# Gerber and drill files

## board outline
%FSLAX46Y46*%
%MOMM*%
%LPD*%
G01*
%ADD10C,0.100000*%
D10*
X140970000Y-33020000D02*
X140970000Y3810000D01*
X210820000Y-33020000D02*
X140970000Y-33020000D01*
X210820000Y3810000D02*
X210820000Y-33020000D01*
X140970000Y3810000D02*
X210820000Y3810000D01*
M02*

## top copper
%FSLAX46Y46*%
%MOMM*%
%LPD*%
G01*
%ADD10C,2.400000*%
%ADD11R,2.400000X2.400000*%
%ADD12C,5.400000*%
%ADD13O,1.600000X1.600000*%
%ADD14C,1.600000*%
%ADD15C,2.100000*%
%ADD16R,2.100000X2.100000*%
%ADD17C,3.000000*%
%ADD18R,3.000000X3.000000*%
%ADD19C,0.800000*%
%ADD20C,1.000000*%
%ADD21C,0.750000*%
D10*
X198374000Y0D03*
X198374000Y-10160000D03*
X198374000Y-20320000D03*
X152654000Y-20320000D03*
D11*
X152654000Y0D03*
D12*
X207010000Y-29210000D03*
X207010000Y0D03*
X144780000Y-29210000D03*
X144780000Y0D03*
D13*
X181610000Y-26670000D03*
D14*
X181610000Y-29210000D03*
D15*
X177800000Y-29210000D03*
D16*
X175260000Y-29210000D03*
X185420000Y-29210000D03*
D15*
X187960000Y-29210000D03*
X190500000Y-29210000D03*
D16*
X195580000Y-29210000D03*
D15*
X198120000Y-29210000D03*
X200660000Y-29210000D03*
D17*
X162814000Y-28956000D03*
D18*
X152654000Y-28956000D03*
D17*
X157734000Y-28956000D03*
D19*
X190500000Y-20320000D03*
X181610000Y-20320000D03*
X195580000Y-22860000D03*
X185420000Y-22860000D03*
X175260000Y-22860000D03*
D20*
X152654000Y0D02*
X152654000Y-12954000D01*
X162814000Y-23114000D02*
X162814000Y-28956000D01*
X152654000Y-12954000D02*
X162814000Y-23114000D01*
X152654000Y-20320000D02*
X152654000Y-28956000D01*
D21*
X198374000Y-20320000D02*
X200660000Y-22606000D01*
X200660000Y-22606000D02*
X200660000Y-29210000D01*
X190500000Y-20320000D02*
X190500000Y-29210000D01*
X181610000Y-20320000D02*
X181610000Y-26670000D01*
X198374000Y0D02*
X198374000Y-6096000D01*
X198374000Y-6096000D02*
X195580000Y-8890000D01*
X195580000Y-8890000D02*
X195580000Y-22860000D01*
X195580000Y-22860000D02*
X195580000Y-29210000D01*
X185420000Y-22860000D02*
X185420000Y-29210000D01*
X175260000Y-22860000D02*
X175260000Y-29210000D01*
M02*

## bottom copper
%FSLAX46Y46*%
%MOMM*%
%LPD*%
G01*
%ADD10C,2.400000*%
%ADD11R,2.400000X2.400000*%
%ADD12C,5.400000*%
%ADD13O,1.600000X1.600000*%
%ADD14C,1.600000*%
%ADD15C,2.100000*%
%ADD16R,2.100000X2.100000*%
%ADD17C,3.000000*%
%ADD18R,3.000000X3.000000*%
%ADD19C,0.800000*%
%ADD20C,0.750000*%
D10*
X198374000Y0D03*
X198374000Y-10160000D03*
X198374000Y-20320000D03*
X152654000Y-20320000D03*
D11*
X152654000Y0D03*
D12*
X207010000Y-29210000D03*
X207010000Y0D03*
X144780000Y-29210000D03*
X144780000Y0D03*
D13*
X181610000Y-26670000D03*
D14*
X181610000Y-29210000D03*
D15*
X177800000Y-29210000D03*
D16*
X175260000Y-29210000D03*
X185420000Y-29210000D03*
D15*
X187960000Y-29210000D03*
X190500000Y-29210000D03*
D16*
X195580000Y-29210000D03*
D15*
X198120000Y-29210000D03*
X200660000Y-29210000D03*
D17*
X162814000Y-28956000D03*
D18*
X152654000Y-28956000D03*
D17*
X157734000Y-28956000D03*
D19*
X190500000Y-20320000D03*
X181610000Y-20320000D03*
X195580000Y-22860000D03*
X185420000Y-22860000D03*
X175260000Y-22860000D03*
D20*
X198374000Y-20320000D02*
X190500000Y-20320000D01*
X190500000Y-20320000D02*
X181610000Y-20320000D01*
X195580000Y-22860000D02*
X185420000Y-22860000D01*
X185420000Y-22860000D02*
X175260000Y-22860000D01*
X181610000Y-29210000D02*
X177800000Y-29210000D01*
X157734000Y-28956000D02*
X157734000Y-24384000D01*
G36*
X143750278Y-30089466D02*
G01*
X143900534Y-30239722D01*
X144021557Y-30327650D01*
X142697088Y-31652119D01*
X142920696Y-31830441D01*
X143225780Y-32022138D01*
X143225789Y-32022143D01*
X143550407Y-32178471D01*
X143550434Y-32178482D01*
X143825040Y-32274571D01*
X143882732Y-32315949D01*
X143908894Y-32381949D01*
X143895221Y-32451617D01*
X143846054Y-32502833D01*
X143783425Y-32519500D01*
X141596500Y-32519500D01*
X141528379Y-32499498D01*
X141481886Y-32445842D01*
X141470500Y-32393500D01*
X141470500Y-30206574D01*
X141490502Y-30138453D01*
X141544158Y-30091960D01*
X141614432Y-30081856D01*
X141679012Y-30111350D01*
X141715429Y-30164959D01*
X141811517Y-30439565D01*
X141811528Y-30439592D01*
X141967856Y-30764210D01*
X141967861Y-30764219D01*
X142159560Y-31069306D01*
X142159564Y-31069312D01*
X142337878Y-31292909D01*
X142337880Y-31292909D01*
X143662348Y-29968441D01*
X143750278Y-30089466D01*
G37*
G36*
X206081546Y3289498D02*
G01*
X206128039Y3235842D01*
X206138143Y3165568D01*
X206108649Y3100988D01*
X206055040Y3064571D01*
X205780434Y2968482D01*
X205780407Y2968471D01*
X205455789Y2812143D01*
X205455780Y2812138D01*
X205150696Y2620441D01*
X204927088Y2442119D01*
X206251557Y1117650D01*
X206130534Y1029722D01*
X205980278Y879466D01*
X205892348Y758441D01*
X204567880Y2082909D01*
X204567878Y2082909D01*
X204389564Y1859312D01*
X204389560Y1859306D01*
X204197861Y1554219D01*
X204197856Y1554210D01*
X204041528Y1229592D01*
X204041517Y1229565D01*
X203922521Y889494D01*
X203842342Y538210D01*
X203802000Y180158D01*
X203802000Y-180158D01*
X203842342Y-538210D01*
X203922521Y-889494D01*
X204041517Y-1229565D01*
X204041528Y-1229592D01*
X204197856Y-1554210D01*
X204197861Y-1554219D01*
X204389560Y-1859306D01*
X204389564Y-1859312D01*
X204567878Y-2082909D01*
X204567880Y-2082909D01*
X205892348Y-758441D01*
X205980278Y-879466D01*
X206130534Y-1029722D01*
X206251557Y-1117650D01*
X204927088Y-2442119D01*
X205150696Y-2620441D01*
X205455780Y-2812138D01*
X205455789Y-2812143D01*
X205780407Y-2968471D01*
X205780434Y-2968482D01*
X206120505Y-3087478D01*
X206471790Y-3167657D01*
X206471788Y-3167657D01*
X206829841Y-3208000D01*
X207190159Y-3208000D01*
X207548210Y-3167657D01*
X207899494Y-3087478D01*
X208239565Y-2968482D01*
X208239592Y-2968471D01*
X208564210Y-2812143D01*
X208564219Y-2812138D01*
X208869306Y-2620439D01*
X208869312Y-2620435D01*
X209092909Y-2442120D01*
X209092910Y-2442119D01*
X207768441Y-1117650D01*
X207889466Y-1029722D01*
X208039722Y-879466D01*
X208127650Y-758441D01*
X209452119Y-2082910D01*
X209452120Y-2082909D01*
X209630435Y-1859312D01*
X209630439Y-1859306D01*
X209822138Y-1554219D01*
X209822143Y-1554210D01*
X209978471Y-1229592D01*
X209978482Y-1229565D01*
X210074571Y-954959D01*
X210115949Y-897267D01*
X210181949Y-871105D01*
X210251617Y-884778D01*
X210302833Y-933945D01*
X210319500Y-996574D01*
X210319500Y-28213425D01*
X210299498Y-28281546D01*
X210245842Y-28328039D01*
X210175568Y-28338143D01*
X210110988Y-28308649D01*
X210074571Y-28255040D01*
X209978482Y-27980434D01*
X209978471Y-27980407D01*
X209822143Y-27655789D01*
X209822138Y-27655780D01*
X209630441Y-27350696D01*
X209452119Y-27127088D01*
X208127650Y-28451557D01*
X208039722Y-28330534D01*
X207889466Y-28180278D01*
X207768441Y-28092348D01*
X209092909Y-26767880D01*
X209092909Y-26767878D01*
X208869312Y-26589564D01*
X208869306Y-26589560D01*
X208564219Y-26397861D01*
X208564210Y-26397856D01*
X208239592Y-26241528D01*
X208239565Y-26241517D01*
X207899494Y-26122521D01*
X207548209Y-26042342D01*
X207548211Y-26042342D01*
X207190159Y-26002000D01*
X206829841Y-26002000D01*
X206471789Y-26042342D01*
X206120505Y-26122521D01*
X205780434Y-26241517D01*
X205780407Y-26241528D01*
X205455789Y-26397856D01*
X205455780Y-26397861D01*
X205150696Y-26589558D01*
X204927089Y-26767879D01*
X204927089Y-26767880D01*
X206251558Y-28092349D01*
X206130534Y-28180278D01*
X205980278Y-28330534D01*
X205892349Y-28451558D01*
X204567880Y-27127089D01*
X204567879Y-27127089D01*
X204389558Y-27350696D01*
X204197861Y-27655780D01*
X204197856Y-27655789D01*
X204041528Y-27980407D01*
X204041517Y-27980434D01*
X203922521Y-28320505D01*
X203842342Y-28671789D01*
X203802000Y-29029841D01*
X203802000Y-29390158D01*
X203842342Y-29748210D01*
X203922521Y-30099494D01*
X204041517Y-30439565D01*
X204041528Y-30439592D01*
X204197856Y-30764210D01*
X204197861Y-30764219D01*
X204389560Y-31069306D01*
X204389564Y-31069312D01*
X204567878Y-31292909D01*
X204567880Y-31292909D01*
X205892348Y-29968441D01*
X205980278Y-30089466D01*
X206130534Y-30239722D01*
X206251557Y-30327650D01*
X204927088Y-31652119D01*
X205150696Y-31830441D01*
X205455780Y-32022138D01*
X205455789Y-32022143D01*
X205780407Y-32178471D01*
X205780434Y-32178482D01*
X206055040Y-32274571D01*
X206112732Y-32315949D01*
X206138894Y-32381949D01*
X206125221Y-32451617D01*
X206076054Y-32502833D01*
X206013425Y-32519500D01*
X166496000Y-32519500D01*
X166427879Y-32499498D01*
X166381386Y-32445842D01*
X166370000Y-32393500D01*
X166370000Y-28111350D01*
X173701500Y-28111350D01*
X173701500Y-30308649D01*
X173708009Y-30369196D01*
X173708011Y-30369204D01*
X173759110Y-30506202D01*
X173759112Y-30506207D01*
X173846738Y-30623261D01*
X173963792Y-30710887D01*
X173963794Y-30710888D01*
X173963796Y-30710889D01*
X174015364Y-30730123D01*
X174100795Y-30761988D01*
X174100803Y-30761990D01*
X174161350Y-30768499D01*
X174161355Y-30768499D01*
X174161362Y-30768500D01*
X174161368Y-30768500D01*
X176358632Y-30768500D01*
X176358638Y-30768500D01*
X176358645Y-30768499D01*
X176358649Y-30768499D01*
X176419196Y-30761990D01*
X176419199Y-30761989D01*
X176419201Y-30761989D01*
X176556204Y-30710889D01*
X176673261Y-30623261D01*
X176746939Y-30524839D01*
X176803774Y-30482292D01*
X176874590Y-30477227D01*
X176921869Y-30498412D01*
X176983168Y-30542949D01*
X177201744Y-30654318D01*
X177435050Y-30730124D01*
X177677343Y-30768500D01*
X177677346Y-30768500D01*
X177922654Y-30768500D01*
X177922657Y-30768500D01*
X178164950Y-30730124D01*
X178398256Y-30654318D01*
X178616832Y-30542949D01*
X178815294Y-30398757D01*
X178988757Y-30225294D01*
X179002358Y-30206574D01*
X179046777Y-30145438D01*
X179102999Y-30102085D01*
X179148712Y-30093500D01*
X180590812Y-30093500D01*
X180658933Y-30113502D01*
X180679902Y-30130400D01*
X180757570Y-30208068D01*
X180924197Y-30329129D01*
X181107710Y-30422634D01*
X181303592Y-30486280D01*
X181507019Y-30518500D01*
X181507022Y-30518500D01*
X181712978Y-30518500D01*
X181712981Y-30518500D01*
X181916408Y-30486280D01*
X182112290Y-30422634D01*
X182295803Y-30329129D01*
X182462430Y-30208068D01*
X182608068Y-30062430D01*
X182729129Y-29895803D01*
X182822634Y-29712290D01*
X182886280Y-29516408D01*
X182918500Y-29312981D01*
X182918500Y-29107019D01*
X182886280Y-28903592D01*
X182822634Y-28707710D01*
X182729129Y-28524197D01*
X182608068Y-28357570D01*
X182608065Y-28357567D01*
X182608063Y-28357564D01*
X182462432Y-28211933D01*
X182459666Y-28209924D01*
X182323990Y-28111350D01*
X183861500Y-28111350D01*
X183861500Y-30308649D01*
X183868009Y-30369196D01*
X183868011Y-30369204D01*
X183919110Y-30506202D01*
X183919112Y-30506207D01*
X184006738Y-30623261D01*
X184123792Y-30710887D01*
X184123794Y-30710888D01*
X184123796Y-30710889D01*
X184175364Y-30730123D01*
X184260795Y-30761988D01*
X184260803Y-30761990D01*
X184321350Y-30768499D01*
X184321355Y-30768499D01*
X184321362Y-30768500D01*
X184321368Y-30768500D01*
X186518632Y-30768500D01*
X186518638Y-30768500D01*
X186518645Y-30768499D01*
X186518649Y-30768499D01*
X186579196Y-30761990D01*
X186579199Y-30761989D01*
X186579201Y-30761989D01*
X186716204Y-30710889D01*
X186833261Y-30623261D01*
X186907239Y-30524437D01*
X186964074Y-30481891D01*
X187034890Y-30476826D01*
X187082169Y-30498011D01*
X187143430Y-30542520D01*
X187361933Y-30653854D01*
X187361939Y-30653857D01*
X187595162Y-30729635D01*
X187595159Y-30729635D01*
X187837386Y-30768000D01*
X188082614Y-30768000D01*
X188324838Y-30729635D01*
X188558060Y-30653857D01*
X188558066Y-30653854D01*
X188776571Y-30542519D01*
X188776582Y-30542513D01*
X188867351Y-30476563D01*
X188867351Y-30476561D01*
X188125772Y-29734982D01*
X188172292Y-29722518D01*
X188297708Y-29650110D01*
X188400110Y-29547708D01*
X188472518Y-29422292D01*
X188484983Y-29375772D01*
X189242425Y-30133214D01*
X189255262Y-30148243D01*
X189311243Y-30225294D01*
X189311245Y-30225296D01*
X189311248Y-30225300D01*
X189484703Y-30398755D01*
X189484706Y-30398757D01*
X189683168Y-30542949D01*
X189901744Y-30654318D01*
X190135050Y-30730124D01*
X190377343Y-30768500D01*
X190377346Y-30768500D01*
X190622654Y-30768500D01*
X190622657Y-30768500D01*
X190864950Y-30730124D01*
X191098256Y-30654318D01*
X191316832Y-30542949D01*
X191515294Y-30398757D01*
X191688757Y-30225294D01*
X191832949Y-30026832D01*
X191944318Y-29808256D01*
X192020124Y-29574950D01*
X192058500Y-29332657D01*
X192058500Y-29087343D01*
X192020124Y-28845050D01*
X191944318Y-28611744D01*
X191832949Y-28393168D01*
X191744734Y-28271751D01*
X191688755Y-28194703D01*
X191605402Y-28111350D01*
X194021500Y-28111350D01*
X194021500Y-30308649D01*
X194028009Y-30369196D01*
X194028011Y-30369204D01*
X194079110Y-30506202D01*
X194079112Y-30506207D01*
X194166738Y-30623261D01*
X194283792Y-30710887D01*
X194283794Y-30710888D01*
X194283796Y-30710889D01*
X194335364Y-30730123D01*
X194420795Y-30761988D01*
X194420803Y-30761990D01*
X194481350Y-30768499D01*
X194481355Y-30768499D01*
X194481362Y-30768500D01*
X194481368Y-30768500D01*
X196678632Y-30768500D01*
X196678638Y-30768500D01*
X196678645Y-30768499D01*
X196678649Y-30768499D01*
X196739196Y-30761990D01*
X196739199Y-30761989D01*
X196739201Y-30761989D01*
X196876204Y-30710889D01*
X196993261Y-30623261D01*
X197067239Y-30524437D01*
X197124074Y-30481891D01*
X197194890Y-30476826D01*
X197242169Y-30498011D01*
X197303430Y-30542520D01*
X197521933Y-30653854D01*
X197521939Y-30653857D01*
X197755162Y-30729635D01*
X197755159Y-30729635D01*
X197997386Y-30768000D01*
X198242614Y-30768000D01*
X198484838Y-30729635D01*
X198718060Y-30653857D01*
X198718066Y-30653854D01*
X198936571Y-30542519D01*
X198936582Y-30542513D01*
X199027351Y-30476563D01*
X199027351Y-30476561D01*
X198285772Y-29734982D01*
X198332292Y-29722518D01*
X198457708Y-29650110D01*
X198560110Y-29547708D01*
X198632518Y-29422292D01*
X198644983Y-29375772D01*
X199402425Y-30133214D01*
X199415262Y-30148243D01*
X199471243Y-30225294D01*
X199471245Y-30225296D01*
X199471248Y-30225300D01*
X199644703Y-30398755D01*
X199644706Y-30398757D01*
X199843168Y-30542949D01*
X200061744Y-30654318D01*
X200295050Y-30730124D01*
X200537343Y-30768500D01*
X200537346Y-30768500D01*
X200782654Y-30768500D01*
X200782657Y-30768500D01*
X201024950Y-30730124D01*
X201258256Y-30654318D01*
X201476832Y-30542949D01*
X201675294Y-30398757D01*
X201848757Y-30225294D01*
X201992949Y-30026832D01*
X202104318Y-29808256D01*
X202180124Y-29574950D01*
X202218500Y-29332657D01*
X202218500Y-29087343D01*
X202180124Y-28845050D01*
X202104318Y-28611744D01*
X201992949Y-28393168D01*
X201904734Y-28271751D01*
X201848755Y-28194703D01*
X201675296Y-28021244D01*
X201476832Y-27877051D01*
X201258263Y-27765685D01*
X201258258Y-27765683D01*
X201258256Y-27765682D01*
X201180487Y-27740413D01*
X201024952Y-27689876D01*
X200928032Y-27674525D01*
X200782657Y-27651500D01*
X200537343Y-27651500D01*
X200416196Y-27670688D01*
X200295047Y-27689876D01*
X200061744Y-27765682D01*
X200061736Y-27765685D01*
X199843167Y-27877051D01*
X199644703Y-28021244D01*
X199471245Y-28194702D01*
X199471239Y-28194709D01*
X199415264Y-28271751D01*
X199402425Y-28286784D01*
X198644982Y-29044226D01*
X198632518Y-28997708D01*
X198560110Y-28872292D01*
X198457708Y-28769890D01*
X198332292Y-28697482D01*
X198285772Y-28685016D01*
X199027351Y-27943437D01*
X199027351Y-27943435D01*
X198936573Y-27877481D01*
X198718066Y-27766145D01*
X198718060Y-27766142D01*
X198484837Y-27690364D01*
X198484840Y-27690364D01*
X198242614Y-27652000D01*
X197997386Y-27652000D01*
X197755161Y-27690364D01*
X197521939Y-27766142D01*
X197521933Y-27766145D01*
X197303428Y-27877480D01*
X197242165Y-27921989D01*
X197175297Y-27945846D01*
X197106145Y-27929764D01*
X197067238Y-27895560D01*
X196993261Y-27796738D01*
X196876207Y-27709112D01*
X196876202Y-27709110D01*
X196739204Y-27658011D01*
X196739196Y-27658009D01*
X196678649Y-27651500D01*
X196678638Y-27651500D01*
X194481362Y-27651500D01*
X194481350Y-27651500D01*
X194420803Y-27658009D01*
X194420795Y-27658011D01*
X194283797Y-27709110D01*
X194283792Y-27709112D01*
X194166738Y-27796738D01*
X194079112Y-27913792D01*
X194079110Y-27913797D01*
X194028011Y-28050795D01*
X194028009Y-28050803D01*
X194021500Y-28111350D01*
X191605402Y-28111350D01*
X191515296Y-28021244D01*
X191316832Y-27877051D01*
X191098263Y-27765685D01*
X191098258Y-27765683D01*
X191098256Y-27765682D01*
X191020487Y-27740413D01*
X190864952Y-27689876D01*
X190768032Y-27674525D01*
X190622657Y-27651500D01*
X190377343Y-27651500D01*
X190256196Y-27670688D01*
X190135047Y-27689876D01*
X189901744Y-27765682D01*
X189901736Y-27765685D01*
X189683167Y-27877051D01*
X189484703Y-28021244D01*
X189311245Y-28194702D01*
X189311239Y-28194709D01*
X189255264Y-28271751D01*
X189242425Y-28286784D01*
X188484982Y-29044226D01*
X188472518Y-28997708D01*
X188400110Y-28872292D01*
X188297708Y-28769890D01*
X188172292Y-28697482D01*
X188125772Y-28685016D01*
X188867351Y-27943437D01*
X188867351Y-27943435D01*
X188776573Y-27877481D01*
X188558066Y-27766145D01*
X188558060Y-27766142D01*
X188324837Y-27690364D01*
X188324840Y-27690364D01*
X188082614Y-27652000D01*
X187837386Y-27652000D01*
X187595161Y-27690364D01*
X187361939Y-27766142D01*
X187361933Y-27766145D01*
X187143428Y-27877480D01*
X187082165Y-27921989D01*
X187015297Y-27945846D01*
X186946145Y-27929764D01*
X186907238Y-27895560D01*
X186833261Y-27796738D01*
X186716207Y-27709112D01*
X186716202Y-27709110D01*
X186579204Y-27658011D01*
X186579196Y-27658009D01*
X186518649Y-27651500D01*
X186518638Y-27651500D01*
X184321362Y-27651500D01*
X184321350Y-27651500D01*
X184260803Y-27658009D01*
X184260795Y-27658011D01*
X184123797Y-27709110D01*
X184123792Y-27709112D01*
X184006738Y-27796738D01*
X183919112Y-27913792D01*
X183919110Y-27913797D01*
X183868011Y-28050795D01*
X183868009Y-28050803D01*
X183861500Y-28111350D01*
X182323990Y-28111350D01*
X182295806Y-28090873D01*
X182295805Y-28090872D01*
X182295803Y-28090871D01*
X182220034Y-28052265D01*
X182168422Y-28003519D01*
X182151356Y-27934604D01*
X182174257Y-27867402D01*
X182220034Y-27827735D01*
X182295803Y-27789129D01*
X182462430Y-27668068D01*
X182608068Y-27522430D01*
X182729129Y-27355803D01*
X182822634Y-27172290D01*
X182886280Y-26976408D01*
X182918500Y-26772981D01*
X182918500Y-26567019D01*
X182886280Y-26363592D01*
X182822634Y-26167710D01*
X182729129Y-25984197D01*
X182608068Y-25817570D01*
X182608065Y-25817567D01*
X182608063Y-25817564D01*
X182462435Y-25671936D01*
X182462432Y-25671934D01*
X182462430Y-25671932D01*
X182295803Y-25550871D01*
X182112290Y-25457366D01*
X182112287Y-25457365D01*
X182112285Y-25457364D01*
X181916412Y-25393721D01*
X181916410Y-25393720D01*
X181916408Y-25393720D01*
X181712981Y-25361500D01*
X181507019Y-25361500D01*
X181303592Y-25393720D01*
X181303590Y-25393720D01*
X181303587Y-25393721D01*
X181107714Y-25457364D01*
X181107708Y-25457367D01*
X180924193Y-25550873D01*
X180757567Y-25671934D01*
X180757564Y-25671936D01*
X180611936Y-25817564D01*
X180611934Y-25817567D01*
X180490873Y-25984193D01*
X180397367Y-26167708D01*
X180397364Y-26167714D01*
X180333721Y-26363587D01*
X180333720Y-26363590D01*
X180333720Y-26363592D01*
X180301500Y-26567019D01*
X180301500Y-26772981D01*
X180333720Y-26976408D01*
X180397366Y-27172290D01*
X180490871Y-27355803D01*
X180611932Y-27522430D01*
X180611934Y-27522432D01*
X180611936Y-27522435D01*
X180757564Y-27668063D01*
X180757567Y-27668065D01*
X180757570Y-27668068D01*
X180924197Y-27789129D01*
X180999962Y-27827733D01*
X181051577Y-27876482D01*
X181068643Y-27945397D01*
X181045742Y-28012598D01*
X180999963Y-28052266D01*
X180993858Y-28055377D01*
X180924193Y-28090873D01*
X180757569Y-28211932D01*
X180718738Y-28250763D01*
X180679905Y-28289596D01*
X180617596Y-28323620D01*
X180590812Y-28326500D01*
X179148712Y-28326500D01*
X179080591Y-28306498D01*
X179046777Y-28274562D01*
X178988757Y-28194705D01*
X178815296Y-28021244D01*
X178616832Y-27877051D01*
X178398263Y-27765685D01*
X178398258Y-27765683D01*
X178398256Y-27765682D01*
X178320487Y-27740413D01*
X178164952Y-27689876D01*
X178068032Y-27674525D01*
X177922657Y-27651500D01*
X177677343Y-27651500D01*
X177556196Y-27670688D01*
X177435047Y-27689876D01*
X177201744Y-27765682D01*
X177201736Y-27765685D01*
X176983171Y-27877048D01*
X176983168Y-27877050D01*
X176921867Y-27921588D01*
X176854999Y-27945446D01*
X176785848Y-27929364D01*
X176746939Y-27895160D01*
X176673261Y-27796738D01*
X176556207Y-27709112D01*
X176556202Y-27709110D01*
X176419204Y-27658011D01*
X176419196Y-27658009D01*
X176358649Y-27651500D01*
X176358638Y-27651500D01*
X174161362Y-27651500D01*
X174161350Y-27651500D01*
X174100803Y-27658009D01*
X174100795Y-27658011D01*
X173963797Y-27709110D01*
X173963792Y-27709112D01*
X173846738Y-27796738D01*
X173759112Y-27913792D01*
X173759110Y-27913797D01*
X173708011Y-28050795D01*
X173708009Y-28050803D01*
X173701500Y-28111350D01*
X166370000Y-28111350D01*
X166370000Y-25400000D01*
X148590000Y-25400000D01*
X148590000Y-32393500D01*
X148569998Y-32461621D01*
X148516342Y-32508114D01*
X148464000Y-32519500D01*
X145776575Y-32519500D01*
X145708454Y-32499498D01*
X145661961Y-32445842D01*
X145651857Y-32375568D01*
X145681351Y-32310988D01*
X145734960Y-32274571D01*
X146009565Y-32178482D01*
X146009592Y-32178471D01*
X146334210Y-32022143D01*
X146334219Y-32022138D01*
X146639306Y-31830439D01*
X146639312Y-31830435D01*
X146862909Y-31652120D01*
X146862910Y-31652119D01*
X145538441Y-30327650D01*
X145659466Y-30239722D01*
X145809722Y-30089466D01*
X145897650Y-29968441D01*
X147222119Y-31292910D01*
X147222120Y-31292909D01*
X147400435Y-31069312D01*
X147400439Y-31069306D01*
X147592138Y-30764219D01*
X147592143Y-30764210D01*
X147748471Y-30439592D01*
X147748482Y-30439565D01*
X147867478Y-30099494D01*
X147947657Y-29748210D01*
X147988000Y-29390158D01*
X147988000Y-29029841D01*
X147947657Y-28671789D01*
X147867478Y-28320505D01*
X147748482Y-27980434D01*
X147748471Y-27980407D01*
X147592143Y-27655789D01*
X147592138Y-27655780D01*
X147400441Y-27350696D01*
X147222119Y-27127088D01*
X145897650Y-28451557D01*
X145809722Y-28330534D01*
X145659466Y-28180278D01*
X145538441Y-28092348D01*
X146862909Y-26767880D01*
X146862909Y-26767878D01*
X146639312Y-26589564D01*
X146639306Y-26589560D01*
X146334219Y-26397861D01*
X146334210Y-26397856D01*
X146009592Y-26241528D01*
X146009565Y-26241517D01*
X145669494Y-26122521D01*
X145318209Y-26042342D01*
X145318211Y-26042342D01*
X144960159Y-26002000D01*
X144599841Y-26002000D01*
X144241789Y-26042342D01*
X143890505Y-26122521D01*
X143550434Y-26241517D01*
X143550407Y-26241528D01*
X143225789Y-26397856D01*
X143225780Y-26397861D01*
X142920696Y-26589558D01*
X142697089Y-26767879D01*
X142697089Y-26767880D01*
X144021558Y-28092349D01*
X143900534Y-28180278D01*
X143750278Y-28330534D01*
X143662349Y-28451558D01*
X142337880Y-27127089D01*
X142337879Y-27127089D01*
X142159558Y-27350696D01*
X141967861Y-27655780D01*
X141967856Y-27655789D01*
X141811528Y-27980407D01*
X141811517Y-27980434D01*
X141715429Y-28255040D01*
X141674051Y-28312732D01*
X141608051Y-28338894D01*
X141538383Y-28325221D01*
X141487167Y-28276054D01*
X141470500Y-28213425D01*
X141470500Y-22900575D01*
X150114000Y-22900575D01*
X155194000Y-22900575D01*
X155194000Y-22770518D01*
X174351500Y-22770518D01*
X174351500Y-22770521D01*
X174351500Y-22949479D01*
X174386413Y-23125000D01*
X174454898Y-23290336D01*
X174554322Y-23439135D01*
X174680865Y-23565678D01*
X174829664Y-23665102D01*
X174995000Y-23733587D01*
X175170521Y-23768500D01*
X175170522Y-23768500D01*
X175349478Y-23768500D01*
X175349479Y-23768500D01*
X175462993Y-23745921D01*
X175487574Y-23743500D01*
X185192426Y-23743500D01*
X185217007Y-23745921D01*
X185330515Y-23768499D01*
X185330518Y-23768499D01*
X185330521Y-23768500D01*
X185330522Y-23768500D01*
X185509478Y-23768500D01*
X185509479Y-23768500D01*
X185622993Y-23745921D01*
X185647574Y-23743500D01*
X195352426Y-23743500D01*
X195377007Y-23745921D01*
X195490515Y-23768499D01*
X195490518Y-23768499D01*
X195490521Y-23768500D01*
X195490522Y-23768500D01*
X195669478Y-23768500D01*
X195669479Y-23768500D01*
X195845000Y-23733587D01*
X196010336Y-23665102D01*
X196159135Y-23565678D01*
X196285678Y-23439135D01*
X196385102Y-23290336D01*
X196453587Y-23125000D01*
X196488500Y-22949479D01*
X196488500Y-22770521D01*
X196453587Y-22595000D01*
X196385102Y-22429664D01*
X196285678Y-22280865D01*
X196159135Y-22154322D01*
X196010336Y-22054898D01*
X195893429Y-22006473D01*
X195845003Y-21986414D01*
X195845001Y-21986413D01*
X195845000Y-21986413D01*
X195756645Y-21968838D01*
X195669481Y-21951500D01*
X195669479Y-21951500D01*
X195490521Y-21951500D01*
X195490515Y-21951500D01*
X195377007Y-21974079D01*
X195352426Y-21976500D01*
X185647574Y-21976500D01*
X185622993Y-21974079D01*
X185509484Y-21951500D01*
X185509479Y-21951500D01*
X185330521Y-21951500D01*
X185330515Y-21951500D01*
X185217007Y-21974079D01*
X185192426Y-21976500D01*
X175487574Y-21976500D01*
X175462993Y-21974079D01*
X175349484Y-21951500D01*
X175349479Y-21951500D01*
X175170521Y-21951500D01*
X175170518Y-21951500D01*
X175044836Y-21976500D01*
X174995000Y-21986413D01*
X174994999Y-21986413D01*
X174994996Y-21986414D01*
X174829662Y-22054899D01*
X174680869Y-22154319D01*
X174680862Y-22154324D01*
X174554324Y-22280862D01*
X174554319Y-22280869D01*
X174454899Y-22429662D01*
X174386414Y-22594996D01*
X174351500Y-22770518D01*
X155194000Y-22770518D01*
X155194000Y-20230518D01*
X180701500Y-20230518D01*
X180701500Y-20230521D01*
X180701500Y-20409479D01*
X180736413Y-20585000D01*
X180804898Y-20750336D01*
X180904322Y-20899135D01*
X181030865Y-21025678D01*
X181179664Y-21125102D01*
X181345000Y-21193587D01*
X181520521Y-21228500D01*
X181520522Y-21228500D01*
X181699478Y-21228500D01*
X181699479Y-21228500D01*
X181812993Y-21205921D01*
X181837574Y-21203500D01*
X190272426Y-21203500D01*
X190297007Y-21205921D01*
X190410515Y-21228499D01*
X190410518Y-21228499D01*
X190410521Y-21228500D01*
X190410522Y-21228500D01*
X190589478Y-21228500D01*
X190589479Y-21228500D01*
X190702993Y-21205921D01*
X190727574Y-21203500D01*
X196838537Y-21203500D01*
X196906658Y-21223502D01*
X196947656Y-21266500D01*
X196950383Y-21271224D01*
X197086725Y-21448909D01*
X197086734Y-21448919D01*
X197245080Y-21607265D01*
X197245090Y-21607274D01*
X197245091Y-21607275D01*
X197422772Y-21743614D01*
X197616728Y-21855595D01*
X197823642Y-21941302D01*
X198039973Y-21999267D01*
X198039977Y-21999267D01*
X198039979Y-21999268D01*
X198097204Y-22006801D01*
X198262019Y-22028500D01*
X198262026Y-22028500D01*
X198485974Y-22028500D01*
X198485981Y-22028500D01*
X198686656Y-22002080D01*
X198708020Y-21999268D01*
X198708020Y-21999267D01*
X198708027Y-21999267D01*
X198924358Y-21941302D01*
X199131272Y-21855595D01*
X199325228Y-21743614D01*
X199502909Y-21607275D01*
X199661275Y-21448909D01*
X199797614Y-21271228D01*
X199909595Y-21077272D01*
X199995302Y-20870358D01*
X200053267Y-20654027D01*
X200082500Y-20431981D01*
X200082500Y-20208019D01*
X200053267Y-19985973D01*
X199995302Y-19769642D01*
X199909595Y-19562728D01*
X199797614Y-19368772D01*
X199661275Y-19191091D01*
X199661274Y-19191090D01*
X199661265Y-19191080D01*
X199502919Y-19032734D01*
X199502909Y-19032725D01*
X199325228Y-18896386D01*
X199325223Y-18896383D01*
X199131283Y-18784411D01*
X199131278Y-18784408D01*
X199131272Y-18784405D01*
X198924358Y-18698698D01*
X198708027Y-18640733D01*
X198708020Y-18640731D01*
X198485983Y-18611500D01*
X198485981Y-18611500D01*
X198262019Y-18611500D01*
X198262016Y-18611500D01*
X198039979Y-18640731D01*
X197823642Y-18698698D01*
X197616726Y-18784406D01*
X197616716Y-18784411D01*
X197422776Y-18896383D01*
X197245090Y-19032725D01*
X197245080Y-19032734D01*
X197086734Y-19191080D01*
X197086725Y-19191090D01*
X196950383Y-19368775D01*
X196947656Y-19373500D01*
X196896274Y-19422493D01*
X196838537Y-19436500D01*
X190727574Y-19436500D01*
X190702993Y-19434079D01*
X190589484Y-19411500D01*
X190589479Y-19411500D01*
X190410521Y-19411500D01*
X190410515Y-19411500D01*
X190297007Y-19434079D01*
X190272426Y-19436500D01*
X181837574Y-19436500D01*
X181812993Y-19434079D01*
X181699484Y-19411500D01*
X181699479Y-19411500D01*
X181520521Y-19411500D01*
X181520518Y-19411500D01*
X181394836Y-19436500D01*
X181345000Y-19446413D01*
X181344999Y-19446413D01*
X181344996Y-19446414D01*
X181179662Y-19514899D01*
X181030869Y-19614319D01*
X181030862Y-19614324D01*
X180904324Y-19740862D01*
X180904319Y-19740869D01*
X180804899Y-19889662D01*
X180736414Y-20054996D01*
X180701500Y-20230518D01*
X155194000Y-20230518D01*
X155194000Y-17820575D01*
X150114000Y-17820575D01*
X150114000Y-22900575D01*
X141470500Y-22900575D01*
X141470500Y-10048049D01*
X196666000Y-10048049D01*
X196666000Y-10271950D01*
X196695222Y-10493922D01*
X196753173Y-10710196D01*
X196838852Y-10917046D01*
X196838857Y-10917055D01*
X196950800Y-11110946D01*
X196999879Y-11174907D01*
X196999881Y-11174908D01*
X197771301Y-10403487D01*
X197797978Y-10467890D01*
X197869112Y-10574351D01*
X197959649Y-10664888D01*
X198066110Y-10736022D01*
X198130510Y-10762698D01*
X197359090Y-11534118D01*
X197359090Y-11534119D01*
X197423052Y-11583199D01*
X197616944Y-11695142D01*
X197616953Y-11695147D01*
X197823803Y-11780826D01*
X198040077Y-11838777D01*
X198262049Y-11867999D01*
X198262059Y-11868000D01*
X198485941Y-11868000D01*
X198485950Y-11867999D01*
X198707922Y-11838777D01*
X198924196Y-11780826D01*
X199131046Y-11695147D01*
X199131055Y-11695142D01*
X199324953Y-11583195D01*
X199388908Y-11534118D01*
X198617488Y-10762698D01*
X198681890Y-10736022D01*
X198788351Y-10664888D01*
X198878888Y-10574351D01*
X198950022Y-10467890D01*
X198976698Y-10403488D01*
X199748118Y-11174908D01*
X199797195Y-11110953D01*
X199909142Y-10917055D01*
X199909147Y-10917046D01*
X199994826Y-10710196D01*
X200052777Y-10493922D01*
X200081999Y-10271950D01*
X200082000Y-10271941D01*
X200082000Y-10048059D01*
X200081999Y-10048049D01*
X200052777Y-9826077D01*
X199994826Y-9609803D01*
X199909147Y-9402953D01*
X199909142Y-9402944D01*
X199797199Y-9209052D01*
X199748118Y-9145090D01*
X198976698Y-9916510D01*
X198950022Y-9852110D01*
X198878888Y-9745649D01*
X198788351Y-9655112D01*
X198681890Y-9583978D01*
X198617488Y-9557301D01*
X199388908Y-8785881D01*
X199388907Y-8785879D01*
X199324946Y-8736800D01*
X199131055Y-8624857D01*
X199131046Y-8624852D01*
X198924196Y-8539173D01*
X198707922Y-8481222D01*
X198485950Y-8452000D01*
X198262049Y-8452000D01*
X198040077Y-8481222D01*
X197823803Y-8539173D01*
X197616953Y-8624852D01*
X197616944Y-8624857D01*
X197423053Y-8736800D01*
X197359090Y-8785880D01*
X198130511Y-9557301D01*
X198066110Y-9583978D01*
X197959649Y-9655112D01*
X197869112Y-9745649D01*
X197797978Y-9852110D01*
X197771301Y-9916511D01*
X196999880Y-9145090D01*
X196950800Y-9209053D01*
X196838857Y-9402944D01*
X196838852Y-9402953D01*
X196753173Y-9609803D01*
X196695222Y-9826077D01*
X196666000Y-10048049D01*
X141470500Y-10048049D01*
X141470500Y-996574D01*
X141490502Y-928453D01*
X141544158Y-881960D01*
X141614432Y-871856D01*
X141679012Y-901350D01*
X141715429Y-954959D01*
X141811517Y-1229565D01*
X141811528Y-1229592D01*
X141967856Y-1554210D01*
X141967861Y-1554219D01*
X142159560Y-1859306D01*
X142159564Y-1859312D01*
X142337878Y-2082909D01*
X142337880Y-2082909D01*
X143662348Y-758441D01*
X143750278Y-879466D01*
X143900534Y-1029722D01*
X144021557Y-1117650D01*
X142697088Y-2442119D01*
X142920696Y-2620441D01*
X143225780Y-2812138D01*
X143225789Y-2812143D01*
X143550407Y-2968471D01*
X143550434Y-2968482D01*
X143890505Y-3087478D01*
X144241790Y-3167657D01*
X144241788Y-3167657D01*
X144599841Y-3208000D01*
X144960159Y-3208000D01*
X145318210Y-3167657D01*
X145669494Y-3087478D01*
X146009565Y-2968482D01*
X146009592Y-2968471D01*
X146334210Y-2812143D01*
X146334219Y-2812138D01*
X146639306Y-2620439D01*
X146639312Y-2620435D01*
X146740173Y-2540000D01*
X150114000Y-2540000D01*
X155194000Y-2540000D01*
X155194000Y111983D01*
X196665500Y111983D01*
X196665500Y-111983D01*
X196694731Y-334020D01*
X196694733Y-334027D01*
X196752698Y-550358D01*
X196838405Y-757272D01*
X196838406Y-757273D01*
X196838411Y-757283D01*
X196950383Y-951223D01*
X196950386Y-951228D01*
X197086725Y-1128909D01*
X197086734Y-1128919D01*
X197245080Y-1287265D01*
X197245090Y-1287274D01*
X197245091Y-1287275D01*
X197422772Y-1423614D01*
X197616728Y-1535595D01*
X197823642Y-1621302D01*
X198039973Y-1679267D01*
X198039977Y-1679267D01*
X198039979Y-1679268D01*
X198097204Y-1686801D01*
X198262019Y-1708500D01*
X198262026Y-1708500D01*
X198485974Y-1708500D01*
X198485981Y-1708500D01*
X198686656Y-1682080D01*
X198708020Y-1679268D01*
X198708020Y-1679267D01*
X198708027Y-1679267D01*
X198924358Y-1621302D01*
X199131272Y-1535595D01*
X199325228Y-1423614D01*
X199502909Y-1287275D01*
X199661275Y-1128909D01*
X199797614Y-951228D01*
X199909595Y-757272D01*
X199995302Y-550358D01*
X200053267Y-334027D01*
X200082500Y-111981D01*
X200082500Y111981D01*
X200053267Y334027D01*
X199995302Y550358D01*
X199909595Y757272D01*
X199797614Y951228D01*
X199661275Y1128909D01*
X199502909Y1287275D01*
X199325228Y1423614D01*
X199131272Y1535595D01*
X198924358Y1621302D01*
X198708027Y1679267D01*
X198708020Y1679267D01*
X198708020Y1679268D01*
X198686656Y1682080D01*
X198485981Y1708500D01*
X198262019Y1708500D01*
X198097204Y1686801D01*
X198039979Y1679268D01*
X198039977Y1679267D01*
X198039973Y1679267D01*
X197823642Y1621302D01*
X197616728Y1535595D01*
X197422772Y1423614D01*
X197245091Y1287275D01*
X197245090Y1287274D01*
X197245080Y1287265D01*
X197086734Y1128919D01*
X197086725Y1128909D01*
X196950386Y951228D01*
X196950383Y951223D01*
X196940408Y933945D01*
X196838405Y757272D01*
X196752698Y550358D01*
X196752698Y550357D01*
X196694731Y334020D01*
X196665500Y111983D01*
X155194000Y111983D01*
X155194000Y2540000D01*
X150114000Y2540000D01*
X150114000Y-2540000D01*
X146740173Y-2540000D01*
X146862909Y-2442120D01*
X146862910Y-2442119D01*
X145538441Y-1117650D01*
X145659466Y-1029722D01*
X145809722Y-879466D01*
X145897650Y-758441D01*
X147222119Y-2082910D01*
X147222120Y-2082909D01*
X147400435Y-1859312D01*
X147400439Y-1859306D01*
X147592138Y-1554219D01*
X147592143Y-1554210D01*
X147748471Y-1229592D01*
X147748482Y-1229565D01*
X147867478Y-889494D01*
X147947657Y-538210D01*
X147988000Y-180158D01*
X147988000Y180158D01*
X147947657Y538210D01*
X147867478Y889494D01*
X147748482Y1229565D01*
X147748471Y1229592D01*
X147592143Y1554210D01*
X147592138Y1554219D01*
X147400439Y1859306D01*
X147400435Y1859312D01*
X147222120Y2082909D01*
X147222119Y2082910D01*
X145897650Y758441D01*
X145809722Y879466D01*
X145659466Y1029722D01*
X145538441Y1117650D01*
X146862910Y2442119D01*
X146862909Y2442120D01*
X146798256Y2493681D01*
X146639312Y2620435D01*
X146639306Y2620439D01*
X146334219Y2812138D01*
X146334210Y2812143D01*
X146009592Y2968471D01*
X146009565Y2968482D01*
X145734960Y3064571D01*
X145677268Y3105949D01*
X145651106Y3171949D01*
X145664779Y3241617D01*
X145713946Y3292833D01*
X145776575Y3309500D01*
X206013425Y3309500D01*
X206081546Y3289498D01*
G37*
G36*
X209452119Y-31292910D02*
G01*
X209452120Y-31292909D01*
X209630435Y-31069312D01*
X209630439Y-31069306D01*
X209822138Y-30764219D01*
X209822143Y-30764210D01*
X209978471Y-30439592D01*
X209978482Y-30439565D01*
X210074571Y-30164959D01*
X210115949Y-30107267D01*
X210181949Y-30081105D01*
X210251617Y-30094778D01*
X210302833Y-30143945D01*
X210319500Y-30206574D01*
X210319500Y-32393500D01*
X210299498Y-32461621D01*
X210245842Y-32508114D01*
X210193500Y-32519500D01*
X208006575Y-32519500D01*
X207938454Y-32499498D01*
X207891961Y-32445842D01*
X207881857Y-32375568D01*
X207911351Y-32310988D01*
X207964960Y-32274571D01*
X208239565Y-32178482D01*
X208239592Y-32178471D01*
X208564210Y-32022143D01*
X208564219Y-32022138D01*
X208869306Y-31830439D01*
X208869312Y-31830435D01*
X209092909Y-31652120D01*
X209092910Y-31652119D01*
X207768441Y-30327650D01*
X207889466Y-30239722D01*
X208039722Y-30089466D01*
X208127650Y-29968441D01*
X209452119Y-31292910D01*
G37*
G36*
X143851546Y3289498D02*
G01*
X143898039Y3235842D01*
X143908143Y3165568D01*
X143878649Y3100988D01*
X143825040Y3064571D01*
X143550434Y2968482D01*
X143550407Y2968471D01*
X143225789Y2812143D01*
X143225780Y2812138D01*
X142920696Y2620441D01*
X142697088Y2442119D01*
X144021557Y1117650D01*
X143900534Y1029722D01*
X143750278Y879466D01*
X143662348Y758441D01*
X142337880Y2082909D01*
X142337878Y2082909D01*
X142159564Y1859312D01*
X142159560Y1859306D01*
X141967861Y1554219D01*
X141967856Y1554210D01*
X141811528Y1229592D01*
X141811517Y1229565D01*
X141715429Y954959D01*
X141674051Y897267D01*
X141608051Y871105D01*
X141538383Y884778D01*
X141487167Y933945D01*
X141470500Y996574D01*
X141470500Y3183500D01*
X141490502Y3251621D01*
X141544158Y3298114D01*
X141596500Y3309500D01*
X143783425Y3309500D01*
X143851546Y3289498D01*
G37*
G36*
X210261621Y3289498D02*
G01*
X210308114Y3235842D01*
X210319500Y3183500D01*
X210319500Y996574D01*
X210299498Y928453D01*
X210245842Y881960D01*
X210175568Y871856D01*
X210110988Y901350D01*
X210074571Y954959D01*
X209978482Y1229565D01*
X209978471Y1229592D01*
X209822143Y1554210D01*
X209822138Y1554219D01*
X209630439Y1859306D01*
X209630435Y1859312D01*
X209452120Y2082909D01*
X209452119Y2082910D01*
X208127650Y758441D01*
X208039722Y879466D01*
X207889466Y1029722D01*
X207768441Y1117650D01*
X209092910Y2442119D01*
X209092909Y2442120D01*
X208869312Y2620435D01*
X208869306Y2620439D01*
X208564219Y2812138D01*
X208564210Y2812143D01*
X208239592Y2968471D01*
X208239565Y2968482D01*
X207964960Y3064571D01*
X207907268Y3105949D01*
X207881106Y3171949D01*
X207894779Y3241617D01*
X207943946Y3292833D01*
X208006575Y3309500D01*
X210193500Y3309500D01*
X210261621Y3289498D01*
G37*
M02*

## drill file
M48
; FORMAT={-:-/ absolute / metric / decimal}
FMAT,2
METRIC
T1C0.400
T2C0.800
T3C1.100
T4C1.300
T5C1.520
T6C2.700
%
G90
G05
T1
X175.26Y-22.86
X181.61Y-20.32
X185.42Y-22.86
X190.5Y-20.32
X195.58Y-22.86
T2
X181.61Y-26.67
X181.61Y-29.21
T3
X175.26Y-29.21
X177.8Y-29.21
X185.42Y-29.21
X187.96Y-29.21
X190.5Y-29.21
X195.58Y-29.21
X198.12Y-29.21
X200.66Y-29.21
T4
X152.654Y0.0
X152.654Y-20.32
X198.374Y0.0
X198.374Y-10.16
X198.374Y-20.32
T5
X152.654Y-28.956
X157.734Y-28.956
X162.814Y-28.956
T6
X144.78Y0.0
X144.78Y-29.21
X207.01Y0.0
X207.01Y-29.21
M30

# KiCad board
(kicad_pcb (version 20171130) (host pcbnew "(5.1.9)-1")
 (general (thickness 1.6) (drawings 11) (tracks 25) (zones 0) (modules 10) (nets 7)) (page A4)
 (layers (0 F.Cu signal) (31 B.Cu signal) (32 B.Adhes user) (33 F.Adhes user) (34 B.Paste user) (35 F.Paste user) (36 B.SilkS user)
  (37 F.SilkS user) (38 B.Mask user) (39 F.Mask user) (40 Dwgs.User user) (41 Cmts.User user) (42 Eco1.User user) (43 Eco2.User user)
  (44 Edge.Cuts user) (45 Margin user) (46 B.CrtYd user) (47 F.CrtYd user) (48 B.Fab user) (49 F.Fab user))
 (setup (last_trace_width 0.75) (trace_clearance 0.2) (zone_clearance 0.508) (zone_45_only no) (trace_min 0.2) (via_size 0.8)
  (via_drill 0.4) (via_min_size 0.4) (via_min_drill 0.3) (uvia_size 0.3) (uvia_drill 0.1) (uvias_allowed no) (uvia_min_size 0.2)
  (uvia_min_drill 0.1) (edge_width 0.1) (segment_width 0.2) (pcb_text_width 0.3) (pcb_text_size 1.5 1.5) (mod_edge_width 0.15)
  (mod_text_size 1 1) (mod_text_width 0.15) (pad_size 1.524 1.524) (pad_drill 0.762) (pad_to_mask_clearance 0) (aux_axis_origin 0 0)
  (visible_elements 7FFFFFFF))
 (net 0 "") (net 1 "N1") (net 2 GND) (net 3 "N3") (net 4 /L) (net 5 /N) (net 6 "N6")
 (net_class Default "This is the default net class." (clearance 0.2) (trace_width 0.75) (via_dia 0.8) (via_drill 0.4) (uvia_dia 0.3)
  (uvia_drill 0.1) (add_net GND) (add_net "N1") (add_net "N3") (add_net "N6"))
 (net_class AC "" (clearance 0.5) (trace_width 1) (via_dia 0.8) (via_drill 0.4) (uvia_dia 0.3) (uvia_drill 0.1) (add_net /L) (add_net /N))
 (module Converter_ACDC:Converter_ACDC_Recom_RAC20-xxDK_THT (layer F.Cu) (at 152.654 0)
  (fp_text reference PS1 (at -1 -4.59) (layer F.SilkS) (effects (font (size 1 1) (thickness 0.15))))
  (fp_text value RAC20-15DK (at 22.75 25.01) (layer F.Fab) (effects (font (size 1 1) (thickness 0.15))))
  (pad 5 thru_hole circle (at 45.72 0) (size 2.4 2.4) (drill 1.3) (layers *.Cu *.Mask) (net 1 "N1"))
  (pad 4 thru_hole circle (at 45.72 10.16) (size 2.4 2.4) (drill 1.3) (layers *.Cu *.Mask) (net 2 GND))
  (pad 3 thru_hole circle (at 45.72 20.32) (size 2.4 2.4) (drill 1.3) (layers *.Cu *.Mask) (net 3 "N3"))
  (pad 2 thru_hole circle (at 0 20.32) (size 2.4 2.4) (drill 1.3) (layers *.Cu *.Mask) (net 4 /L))
  (pad 1 thru_hole rect (at 0 0) (size 2.4 2.4) (drill 1.3) (layers *.Cu *.Mask) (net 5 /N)))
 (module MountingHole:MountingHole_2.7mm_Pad (layer F.Cu) (at 207.01 29.21)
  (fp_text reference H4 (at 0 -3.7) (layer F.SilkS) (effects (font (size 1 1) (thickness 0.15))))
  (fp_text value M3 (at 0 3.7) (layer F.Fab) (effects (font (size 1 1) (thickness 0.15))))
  (pad 1 thru_hole circle (at 0 0) (size 5.4 5.4) (drill 2.7) (layers *.Cu *.Mask) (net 2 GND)))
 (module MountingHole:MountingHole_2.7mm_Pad (layer F.Cu) (at 207.01 0)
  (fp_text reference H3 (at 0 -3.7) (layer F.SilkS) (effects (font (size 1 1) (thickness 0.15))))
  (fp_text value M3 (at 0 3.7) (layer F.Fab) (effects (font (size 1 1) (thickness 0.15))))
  (pad 1 thru_hole circle (at 0 0) (size 5.4 5.4) (drill 2.7) (layers *.Cu *.Mask) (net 2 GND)))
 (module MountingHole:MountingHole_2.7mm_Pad (layer F.Cu) (at 144.78 29.21)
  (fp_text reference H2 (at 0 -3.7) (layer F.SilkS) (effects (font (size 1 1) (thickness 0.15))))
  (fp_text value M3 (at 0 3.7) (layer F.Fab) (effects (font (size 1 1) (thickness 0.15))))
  (pad 1 thru_hole circle (at 0 0) (size 5.4 5.4) (drill 2.7) (layers *.Cu *.Mask) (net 2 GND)))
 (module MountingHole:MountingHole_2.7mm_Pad (layer F.Cu) (at 144.78 0)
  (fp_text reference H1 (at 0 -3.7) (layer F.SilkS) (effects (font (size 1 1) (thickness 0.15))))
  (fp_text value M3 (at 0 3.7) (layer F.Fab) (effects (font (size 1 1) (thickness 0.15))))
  (pad 1 thru_hole circle (at 0 0) (size 5.4 5.4) (drill 2.7) (layers *.Cu *.Mask) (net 2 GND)))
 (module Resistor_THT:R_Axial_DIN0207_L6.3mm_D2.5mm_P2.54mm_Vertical (layer F.Cu) (at 181.61 29.21 90)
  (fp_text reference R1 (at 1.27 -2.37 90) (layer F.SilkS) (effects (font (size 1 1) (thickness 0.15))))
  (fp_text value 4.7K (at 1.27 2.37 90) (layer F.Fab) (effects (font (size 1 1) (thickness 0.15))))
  (pad 2 thru_hole oval (at 2.54 0 90) (size 1.6 1.6) (drill 0.8) (layers *.Cu *.Mask) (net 3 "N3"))
  (pad 1 thru_hole circle (at 0 0 90) (size 1.6 1.6) (drill 0.8) (layers *.Cu *.Mask) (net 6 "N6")))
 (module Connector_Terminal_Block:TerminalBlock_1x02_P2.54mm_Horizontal (layer F.Cu) (at 175.26 29.21)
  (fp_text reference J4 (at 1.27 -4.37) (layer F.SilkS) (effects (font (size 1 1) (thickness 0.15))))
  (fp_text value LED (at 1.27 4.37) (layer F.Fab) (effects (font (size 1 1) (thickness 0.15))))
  (pad 2 thru_hole circle (at 2.54 0) (size 2.1 2.1) (drill 1.1) (layers *.Cu *.Mask) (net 6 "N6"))
  (pad 1 thru_hole rect (at 0 0) (size 2.1 2.1) (drill 1.1) (layers *.Cu *.Mask) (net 1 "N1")))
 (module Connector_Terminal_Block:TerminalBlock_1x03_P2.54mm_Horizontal (layer F.Cu) (at 185.42 29.21)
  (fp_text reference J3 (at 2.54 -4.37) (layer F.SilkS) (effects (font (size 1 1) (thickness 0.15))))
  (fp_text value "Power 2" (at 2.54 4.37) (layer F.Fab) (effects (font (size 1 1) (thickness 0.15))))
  (pad 1 thru_hole rect (at 0 0) (size 2.1 2.1) (drill 1.1) (layers *.Cu *.Mask) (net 1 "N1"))
  (pad 2 thru_hole circle (at 2.54 0) (size 2.1 2.1) (drill 1.1) (layers *.Cu *.Mask) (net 2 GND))
  (pad 3 thru_hole circle (at 5.08 0) (size 2.1 2.1) (drill 1.1) (layers *.Cu *.Mask) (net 3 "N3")))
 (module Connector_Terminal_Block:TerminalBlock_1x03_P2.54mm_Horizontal (layer F.Cu) (at 195.58 29.21)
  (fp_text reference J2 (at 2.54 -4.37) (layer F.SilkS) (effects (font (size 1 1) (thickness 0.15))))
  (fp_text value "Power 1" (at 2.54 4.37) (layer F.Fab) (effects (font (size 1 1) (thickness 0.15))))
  (pad 1 thru_hole rect (at 0 0) (size 2.1 2.1) (drill 1.1) (layers *.Cu *.Mask) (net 1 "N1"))
  (pad 2 thru_hole circle (at 2.54 0) (size 2.1 2.1) (drill 1.1) (layers *.Cu *.Mask) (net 2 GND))
  (pad 3 thru_hole circle (at 5.08 0) (size 2.1 2.1) (drill 1.1) (layers *.Cu *.Mask) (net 3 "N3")))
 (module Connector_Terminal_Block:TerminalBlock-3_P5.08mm (layer F.Cu) (at 152.654 28.956)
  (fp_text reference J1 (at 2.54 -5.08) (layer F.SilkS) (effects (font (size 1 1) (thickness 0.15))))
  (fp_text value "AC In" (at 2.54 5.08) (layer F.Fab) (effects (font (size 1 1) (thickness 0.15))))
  (pad 3 thru_hole circle (at 10.16 0) (size 3 3) (drill 1.52) (layers *.Cu *.Mask) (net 5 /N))
  (pad 1 thru_hole rect (at 0 0) (size 3 3) (drill 1.52) (layers *.Cu *.Mask) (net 4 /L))
  (pad 2 thru_hole circle (at 5.08 0) (size 3 3) (drill 1.52) (layers *.Cu *.Mask) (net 2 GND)))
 (gr_line (start 140.97 33.02) (end 140.97 -3.81) (layer Edge.Cuts) (width 0.1))
 (gr_line (start 210.82 33.02) (end 140.97 33.02) (layer Edge.Cuts) (width 0.1))
 (gr_line (start 210.82 -3.81) (end 210.82 33.02) (layer Edge.Cuts) (width 0.1))
 (gr_line (start 140.97 -3.81) (end 210.82 -3.81) (layer Edge.Cuts) (width 0.1))
 (segment (start 152.654 0) (end 152.654 12.954) (width 1) (layer F.Cu) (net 5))
 (segment (start 162.814 23.114) (end 162.814 28.956) (width 1) (layer F.Cu) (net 5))
 (segment (start 152.654 12.954) (end 162.814 23.114) (width 1) (layer F.Cu) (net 5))
 (segment (start 152.654 20.32) (end 152.654 28.956) (width 1) (layer F.Cu) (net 4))
 (segment (start 198.374 20.32) (end 200.66 22.606) (width 0.75) (layer F.Cu) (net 3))
 (segment (start 200.66 22.606) (end 200.66 29.21) (width 0.75) (layer F.Cu) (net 3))
 (via (at 190.5 20.32) (size 0.8) (drill 0.4) (layers F.Cu B.Cu) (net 3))
 (segment (start 198.374 20.32) (end 190.5 20.32) (width 0.75) (layer B.Cu) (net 3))
 (segment (start 190.5 20.32) (end 190.5 29.21) (width 0.75) (layer F.Cu) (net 3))
 (via (at 181.61 20.32) (size 0.8) (drill 0.4) (layers F.Cu B.Cu) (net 3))
 (segment (start 190.5 20.32) (end 181.61 20.32) (width 0.75) (layer B.Cu) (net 3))
 (segment (start 181.61 20.32) (end 181.61 26.67) (width 0.75) (layer F.Cu) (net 3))
 (segment (start 198.374 0) (end 198.374 6.096) (width 0.75) (layer F.Cu) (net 1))
 (segment (start 198.374 6.096) (end 195.58 8.89) (width 0.75) (layer F.Cu) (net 1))
 (via (at 195.58 22.86) (size 0.8) (drill 0.4) (layers F.Cu B.Cu) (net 1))
 (segment (start 195.58 8.89) (end 195.58 22.86) (width 0.75) (layer F.Cu) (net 1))
 (segment (start 195.58 22.86) (end 195.58 29.21) (width 0.75) (layer F.Cu) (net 1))
 (segment (start 195.58 22.86) (end 185.42 22.86) (width 0.75) (layer B.Cu) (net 1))
 (via (at 185.42 22.86) (size 0.8) (drill 0.4) (layers F.Cu B.Cu) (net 1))
 (segment (start 185.42 22.86) (end 185.42 29.21) (width 0.75) (layer F.Cu) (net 1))
 (via (at 175.26 22.86) (size 0.8) (drill 0.4) (layers F.Cu B.Cu) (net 1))
 (segment (start 185.42 22.86) (end 175.26 22.86) (width 0.75) (layer B.Cu) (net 1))
 (segment (start 175.26 22.86) (end 175.26 29.21) (width 0.75) (layer F.Cu) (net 1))
 (segment (start 181.61 29.21) (end 177.8 29.21) (width 0.75) (layer B.Cu) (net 6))
 (segment (start 157.734 28.956) (end 157.734 24.384) (width 0.75) (layer B.Cu) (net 2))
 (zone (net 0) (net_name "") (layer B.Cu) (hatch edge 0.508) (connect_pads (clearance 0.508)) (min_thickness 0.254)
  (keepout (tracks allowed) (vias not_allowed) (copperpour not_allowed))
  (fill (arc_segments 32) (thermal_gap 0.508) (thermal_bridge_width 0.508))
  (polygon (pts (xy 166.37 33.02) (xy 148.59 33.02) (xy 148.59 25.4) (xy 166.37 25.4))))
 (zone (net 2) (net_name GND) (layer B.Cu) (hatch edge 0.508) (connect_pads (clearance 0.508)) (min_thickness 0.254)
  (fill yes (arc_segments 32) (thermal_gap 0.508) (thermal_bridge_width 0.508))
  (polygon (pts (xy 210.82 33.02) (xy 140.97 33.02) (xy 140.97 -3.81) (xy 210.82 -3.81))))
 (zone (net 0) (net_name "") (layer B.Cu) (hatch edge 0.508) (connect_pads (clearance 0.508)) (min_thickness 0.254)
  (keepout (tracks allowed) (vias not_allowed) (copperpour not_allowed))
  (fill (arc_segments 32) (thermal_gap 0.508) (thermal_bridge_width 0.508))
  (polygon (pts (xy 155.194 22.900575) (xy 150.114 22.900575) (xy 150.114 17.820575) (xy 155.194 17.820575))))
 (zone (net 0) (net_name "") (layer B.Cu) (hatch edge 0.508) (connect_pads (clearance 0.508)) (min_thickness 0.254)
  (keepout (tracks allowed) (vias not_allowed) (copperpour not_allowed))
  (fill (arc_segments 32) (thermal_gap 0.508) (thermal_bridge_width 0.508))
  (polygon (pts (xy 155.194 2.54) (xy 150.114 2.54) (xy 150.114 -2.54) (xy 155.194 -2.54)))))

